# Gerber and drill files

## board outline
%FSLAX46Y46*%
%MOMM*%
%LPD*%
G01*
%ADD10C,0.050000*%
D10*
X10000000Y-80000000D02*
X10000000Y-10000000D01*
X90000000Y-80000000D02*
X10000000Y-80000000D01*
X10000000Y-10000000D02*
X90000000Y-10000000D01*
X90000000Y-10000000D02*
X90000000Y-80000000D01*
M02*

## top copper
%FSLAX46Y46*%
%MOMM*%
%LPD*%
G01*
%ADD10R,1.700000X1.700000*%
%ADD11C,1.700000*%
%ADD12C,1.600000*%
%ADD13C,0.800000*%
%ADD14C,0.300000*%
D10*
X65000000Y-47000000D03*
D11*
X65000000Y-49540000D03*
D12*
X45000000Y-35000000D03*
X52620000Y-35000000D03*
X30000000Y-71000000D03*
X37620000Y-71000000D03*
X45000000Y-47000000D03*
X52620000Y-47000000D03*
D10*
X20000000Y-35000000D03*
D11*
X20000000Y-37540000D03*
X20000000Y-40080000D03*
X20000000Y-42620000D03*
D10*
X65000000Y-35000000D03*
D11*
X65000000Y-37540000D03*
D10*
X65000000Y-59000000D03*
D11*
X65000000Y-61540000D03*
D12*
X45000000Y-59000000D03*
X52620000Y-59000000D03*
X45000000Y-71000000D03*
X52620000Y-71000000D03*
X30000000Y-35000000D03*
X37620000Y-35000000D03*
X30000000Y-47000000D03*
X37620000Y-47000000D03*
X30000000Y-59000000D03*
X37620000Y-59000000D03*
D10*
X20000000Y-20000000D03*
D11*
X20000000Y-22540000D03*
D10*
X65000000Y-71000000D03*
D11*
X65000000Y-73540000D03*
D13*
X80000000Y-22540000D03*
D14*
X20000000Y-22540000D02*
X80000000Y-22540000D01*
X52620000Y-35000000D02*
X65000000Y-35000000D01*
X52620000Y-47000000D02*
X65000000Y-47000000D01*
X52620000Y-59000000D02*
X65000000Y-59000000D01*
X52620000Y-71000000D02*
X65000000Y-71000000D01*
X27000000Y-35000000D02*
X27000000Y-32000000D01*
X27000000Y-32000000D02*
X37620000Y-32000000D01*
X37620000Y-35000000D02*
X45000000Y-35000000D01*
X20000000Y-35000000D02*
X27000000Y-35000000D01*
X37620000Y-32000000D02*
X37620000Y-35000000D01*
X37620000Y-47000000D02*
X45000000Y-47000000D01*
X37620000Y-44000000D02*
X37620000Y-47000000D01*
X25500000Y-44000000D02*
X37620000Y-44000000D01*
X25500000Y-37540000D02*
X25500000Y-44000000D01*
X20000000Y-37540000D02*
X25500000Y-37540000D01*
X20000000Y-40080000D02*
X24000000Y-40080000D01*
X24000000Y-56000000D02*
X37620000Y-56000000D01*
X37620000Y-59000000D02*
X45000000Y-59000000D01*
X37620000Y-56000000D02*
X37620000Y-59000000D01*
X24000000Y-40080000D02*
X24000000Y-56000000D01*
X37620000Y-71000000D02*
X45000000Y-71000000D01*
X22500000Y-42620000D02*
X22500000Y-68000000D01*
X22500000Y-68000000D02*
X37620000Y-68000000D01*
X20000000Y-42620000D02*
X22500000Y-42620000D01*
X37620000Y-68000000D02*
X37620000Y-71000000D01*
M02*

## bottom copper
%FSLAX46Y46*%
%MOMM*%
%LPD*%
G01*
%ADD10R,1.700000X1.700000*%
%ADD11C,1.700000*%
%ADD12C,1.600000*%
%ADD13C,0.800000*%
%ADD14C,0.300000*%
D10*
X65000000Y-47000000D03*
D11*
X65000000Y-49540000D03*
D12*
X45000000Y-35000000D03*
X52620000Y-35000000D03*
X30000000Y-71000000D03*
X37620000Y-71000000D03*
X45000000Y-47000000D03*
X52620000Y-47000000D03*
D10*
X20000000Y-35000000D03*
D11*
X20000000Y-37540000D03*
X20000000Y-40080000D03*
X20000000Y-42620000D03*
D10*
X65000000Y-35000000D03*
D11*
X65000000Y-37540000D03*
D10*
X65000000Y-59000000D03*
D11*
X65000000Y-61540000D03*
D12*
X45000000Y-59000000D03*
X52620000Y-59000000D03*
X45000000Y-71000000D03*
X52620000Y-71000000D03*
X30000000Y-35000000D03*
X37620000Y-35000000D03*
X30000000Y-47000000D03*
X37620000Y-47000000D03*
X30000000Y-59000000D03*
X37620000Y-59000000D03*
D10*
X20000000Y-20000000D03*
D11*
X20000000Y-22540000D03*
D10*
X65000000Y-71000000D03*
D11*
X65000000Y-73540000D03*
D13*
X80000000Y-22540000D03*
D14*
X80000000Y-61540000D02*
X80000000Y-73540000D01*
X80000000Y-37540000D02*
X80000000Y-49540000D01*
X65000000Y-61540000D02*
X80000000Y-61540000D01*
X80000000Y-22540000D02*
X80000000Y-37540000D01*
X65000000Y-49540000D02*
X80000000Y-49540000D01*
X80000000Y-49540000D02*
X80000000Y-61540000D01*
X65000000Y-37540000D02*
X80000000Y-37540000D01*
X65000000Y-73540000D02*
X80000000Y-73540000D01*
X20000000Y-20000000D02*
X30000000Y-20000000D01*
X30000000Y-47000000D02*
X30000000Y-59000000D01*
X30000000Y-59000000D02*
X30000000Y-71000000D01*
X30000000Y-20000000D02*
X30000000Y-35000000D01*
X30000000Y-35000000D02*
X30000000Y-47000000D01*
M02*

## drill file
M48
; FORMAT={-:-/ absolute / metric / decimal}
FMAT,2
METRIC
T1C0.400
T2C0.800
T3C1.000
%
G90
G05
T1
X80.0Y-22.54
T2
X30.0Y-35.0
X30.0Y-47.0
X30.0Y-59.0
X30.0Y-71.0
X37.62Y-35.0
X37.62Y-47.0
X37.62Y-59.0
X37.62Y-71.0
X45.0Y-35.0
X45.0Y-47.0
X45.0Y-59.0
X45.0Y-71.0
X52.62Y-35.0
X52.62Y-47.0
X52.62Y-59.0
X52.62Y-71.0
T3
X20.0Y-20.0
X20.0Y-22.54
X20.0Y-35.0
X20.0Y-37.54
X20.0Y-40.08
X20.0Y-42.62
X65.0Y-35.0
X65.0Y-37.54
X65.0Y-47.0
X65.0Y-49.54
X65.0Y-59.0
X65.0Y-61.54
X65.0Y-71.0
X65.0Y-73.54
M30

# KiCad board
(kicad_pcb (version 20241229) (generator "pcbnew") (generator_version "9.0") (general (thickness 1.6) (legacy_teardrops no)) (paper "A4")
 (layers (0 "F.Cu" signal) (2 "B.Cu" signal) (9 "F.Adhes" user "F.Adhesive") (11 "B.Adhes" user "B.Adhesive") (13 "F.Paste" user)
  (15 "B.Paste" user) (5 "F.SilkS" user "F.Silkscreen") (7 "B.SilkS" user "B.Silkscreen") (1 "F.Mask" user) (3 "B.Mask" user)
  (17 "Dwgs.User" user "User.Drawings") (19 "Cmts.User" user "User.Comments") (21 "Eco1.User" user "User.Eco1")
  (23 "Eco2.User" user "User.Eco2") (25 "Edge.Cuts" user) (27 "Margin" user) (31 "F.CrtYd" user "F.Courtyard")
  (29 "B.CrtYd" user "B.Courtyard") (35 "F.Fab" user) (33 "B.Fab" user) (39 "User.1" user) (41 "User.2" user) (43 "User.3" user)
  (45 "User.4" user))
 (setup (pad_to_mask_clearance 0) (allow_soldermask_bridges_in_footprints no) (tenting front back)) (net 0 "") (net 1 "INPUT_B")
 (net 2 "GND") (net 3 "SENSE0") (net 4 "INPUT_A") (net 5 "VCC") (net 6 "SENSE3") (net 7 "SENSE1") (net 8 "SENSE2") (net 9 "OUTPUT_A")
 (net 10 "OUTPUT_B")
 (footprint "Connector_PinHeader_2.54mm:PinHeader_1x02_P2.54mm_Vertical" (layer "F.Cu") (at 65 47)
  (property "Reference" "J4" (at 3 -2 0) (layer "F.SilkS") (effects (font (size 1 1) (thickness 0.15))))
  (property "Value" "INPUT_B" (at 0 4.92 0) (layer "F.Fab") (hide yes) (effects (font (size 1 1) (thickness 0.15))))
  (pad "1" thru_hole rect (at 0 0) (size 1.7 1.7) (drill 1) (layers "*.Cu" "*.Mask") (remove_unused_layers no) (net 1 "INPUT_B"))
  (pad "2" thru_hole circle (at 0 2.54) (size 1.7 1.7) (drill 1) (layers "*.Cu" "*.Mask") (remove_unused_layers no) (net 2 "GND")))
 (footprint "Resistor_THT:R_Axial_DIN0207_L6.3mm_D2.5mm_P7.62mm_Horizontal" (layer "F.Cu") (at 45 35)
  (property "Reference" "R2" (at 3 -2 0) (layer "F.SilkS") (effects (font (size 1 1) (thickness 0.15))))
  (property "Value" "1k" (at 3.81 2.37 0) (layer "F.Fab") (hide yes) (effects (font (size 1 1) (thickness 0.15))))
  (pad "1" thru_hole circle (at 0 0) (size 1.6 1.6) (drill 0.8) (layers "*.Cu" "*.Mask") (remove_unused_layers no) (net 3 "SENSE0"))
  (pad "2" thru_hole circle (at 7.62 0) (size 1.6 1.6) (drill 0.8) (layers "*.Cu" "*.Mask") (remove_unused_layers no) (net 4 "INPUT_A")))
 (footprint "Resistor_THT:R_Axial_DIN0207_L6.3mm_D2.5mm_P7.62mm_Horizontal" (layer "F.Cu") (at 30 71)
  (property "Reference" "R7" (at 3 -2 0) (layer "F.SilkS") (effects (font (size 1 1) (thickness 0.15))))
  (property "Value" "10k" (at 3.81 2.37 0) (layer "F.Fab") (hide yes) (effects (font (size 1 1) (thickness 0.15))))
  (pad "1" thru_hole circle (at 0 0) (size 1.6 1.6) (drill 0.8) (layers "*.Cu" "*.Mask") (remove_unused_layers no) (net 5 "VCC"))
  (pad "2" thru_hole circle (at 7.62 0) (size 1.6 1.6) (drill 0.8) (layers "*.Cu" "*.Mask") (remove_unused_layers no) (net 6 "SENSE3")))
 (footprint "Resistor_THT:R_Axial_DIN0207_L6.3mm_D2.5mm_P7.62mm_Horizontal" (layer "F.Cu") (at 45 47)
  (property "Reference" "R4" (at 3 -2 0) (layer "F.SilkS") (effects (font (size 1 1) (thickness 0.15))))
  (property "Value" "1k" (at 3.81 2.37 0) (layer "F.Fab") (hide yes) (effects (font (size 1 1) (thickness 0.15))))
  (pad "1" thru_hole circle (at 0 0) (size 1.6 1.6) (drill 0.8) (layers "*.Cu" "*.Mask") (remove_unused_layers no) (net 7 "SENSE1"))
  (pad "2" thru_hole circle (at 7.62 0) (size 1.6 1.6) (drill 0.8) (layers "*.Cu" "*.Mask") (remove_unused_layers no) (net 1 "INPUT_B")))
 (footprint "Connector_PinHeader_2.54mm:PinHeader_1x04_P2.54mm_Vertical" (layer "F.Cu") (at 20 35)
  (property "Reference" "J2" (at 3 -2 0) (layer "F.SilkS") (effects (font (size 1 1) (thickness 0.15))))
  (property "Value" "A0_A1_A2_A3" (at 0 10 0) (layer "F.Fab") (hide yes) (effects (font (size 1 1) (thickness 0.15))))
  (pad "1" thru_hole rect (at 0 0) (size 1.7 1.7) (drill 1) (layers "*.Cu" "*.Mask") (remove_unused_layers no) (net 3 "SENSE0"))
  (pad "2" thru_hole circle (at 0 2.54) (size 1.7 1.7) (drill 1) (layers "*.Cu" "*.Mask") (remove_unused_layers no) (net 7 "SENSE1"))
  (pad "3" thru_hole circle (at 0 5.08) (size 1.7 1.7) (drill 1) (layers "*.Cu" "*.Mask") (remove_unused_layers no) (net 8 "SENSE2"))
  (pad "4" thru_hole circle (at 0 7.62) (size 1.7 1.7) (drill 1) (layers "*.Cu" "*.Mask") (remove_unused_layers no) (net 6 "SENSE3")))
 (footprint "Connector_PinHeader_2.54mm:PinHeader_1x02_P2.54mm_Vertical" (layer "F.Cu") (at 65 35)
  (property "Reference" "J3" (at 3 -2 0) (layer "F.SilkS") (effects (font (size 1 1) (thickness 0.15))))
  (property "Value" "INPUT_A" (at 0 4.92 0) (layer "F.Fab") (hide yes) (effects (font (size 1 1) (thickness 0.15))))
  (pad "1" thru_hole rect (at 0 0) (size 1.7 1.7) (drill 1) (layers "*.Cu" "*.Mask") (remove_unused_layers no) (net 4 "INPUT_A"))
  (pad "2" thru_hole circle (at 0 2.54) (size 1.7 1.7) (drill 1) (layers "*.Cu" "*.Mask") (remove_unused_layers no) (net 2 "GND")))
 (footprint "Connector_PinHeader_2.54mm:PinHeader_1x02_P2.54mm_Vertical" (layer "F.Cu") (at 65 59)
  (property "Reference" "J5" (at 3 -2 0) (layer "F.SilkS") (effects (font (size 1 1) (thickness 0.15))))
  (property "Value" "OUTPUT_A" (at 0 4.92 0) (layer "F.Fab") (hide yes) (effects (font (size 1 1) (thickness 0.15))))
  (pad "1" thru_hole rect (at 0 0) (size 1.7 1.7) (drill 1) (layers "*.Cu" "*.Mask") (remove_unused_layers no) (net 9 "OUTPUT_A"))
  (pad "2" thru_hole circle (at 0 2.54) (size 1.7 1.7) (drill 1) (layers "*.Cu" "*.Mask") (remove_unused_layers no) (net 2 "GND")))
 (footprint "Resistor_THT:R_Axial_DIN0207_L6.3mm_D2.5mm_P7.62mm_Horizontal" (layer "F.Cu") (at 45 59)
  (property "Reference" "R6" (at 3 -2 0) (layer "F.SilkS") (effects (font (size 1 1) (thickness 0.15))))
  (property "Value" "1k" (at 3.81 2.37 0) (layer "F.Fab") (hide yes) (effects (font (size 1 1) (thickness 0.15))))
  (pad "1" thru_hole circle (at 0 0) (size 1.6 1.6) (drill 0.8) (layers "*.Cu" "*.Mask") (remove_unused_layers no) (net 8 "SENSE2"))
  (pad "2" thru_hole circle (at 7.62 0) (size 1.6 1.6) (drill 0.8) (layers "*.Cu" "*.Mask") (remove_unused_layers no) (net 9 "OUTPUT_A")))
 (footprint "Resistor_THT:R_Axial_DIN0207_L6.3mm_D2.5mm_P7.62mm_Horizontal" (layer "F.Cu") (at 45 71)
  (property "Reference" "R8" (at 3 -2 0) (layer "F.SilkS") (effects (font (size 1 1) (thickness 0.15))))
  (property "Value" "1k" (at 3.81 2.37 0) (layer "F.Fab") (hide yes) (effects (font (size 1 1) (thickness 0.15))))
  (pad "1" thru_hole circle (at 0 0) (size 1.6 1.6) (drill 0.8) (layers "*.Cu" "*.Mask") (remove_unused_layers no) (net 6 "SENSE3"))
  (pad "2" thru_hole circle (at 7.62 0) (size 1.6 1.6) (drill 0.8) (layers "*.Cu" "*.Mask") (remove_unused_layers no) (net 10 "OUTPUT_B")))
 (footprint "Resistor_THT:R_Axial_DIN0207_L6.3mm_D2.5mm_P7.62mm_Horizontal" (layer "F.Cu") (at 30 35)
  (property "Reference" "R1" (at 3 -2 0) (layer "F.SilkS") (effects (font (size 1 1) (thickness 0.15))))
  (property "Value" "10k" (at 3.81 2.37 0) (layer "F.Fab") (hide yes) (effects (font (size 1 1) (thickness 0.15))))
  (pad "1" thru_hole circle (at 0 0) (size 1.6 1.6) (drill 0.8) (layers "*.Cu" "*.Mask") (remove_unused_layers no) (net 5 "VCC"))
  (pad "2" thru_hole circle (at 7.62 0) (size 1.6 1.6) (drill 0.8) (layers "*.Cu" "*.Mask") (remove_unused_layers no) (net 3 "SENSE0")))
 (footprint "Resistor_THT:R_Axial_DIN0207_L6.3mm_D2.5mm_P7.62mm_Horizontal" (layer "F.Cu") (at 30 47)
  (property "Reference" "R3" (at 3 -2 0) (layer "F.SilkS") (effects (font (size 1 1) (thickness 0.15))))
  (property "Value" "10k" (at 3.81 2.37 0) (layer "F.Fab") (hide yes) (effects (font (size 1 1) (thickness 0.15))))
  (pad "1" thru_hole circle (at 0 0) (size 1.6 1.6) (drill 0.8) (layers "*.Cu" "*.Mask") (remove_unused_layers no) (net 5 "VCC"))
  (pad "2" thru_hole circle (at 7.62 0) (size 1.6 1.6) (drill 0.8) (layers "*.Cu" "*.Mask") (remove_unused_layers no) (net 7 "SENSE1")))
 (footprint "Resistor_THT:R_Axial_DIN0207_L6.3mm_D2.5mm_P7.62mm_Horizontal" (layer "F.Cu") (at 30 59)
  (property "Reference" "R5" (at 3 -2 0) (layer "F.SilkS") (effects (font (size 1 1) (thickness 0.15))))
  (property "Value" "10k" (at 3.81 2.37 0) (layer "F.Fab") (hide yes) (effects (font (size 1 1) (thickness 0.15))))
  (pad "1" thru_hole circle (at 0 0) (size 1.6 1.6) (drill 0.8) (layers "*.Cu" "*.Mask") (remove_unused_layers no) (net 5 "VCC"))
  (pad "2" thru_hole circle (at 7.62 0) (size 1.6 1.6) (drill 0.8) (layers "*.Cu" "*.Mask") (remove_unused_layers no) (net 8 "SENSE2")))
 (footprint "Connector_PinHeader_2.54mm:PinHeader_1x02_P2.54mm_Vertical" (layer "F.Cu") (at 20 20)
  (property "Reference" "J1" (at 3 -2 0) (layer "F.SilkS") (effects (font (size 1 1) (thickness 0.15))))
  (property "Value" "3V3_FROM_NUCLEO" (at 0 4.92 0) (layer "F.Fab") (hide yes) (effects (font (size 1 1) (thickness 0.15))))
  (pad "1" thru_hole rect (at 0 0) (size 1.7 1.7) (drill 1) (layers "*.Cu" "*.Mask") (remove_unused_layers no) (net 5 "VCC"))
  (pad "2" thru_hole circle (at 0 2.54) (size 1.7 1.7) (drill 1) (layers "*.Cu" "*.Mask") (remove_unused_layers no) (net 2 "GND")))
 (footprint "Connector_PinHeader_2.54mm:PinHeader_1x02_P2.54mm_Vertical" (layer "F.Cu") (at 65 71)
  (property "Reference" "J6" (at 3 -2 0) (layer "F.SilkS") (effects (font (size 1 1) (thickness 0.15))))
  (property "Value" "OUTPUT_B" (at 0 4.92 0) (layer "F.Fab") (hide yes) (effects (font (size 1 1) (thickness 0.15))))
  (pad "1" thru_hole rect (at 0 0) (size 1.7 1.7) (drill 1) (layers "*.Cu" "*.Mask") (remove_unused_layers no) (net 10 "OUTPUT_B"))
  (pad "2" thru_hole circle (at 0 2.54) (size 1.7 1.7) (drill 1) (layers "*.Cu" "*.Mask") (remove_unused_layers no) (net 2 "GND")))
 (gr_line (start 10 80) (end 10 10) (stroke (width 0.05) (type default)) (layer "Edge.Cuts"))
 (gr_line (start 90 80) (end 10 80) (stroke (width 0.05) (type default)) (layer "Edge.Cuts"))
 (gr_line (start 10 10) (end 90 10) (stroke (width 0.05) (type default)) (layer "Edge.Cuts"))
 (gr_line (start 90 10) (end 90 80) (stroke (width 0.05) (type default)) (layer "Edge.Cuts"))
 (segment (start 20 22.54) (end 80 22.54) (width 0.3) (layer "F.Cu") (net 2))
 (via (at 80 22.54) (size 0.8) (drill 0.4) (layers "F.Cu" "B.Cu") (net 2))
 (segment (start 80 61.54) (end 80 73.54) (width 0.3) (layer "B.Cu") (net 2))
 (segment (start 80 37.54) (end 80 49.54) (width 0.3) (layer "B.Cu") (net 2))
 (segment (start 65 61.54) (end 80 61.54) (width 0.3) (layer "B.Cu") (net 2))
 (segment (start 80 22.54) (end 80 37.54) (width 0.3) (layer "B.Cu") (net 2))
 (segment (start 65 49.54) (end 80 49.54) (width 0.3) (layer "B.Cu") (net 2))
 (segment (start 80 49.54) (end 80 61.54) (width 0.3) (layer "B.Cu") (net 2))
 (segment (start 65 37.54) (end 80 37.54) (width 0.3) (layer "B.Cu") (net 2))
 (segment (start 65 73.54) (end 80 73.54) (width 0.3) (layer "B.Cu") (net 2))
 (segment (start 52.62 35) (end 65 35) (width 0.3) (layer "F.Cu") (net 4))
 (segment (start 52.62 47) (end 65 47) (width 0.3) (layer "F.Cu") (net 1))
 (segment (start 52.62 59) (end 65 59) (width 0.3) (layer "F.Cu") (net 9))
 (segment (start 52.62 71) (end 65 71) (width 0.3) (layer "F.Cu") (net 10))
 (segment (start 27 35) (end 27 32) (width 0.3) (layer "F.Cu") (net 3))
 (segment (start 27 32) (end 37.62 32) (width 0.3) (layer "F.Cu") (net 3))
 (segment (start 37.62 35) (end 45 35) (width 0.3) (layer "F.Cu") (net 3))
 (segment (start 20 35) (end 27 35) (width 0.3) (layer "F.Cu") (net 3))
 (segment (start 37.62 32) (end 37.62 35) (width 0.3) (layer "F.Cu") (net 3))
 (segment (start 37.62 47) (end 45 47) (width 0.3) (layer "F.Cu") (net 7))
 (segment (start 37.62 44) (end 37.62 47) (width 0.3) (layer "F.Cu") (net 7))
 (segment (start 25.5 44) (end 37.62 44) (width 0.3) (layer "F.Cu") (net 7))
 (segment (start 25.5 37.54) (end 25.5 44) (width 0.3) (layer "F.Cu") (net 7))
 (segment (start 20 37.54) (end 25.5 37.54) (width 0.3) (layer "F.Cu") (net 7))
 (segment (start 20 40.08) (end 24 40.08) (width 0.3) (layer "F.Cu") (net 8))
 (segment (start 24 56) (end 37.62 56) (width 0.3) (layer "F.Cu") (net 8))
 (segment (start 37.62 59) (end 45 59) (width 0.3) (layer "F.Cu") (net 8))
 (segment (start 37.62 56) (end 37.62 59) (width 0.3) (layer "F.Cu") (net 8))
 (segment (start 24 40.08) (end 24 56) (width 0.3) (layer "F.Cu") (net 8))
 (segment (start 37.62 71) (end 45 71) (width 0.3) (layer "F.Cu") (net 6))
 (segment (start 22.5 42.62) (end 22.5 68) (width 0.3) (layer "F.Cu") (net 6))
 (segment (start 22.5 68) (end 37.62 68) (width 0.3) (layer "F.Cu") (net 6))
 (segment (start 20 42.62) (end 22.5 42.62) (width 0.3) (layer "F.Cu") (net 6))
 (segment (start 37.62 68) (end 37.62 71) (width 0.3) (layer "F.Cu") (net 6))
 (segment (start 20 20) (end 30 20) (width 0.3) (layer "B.Cu") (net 5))
 (segment (start 30 47) (end 30 59) (width 0.3) (layer "B.Cu") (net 5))
 (segment (start 30 59) (end 30 71) (width 0.3) (layer "B.Cu") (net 5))
 (segment (start 30 20) (end 30 35) (width 0.3) (layer "B.Cu") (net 5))
 (segment (start 30 35) (end 30 47) (width 0.3) (layer "B.Cu") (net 5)))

